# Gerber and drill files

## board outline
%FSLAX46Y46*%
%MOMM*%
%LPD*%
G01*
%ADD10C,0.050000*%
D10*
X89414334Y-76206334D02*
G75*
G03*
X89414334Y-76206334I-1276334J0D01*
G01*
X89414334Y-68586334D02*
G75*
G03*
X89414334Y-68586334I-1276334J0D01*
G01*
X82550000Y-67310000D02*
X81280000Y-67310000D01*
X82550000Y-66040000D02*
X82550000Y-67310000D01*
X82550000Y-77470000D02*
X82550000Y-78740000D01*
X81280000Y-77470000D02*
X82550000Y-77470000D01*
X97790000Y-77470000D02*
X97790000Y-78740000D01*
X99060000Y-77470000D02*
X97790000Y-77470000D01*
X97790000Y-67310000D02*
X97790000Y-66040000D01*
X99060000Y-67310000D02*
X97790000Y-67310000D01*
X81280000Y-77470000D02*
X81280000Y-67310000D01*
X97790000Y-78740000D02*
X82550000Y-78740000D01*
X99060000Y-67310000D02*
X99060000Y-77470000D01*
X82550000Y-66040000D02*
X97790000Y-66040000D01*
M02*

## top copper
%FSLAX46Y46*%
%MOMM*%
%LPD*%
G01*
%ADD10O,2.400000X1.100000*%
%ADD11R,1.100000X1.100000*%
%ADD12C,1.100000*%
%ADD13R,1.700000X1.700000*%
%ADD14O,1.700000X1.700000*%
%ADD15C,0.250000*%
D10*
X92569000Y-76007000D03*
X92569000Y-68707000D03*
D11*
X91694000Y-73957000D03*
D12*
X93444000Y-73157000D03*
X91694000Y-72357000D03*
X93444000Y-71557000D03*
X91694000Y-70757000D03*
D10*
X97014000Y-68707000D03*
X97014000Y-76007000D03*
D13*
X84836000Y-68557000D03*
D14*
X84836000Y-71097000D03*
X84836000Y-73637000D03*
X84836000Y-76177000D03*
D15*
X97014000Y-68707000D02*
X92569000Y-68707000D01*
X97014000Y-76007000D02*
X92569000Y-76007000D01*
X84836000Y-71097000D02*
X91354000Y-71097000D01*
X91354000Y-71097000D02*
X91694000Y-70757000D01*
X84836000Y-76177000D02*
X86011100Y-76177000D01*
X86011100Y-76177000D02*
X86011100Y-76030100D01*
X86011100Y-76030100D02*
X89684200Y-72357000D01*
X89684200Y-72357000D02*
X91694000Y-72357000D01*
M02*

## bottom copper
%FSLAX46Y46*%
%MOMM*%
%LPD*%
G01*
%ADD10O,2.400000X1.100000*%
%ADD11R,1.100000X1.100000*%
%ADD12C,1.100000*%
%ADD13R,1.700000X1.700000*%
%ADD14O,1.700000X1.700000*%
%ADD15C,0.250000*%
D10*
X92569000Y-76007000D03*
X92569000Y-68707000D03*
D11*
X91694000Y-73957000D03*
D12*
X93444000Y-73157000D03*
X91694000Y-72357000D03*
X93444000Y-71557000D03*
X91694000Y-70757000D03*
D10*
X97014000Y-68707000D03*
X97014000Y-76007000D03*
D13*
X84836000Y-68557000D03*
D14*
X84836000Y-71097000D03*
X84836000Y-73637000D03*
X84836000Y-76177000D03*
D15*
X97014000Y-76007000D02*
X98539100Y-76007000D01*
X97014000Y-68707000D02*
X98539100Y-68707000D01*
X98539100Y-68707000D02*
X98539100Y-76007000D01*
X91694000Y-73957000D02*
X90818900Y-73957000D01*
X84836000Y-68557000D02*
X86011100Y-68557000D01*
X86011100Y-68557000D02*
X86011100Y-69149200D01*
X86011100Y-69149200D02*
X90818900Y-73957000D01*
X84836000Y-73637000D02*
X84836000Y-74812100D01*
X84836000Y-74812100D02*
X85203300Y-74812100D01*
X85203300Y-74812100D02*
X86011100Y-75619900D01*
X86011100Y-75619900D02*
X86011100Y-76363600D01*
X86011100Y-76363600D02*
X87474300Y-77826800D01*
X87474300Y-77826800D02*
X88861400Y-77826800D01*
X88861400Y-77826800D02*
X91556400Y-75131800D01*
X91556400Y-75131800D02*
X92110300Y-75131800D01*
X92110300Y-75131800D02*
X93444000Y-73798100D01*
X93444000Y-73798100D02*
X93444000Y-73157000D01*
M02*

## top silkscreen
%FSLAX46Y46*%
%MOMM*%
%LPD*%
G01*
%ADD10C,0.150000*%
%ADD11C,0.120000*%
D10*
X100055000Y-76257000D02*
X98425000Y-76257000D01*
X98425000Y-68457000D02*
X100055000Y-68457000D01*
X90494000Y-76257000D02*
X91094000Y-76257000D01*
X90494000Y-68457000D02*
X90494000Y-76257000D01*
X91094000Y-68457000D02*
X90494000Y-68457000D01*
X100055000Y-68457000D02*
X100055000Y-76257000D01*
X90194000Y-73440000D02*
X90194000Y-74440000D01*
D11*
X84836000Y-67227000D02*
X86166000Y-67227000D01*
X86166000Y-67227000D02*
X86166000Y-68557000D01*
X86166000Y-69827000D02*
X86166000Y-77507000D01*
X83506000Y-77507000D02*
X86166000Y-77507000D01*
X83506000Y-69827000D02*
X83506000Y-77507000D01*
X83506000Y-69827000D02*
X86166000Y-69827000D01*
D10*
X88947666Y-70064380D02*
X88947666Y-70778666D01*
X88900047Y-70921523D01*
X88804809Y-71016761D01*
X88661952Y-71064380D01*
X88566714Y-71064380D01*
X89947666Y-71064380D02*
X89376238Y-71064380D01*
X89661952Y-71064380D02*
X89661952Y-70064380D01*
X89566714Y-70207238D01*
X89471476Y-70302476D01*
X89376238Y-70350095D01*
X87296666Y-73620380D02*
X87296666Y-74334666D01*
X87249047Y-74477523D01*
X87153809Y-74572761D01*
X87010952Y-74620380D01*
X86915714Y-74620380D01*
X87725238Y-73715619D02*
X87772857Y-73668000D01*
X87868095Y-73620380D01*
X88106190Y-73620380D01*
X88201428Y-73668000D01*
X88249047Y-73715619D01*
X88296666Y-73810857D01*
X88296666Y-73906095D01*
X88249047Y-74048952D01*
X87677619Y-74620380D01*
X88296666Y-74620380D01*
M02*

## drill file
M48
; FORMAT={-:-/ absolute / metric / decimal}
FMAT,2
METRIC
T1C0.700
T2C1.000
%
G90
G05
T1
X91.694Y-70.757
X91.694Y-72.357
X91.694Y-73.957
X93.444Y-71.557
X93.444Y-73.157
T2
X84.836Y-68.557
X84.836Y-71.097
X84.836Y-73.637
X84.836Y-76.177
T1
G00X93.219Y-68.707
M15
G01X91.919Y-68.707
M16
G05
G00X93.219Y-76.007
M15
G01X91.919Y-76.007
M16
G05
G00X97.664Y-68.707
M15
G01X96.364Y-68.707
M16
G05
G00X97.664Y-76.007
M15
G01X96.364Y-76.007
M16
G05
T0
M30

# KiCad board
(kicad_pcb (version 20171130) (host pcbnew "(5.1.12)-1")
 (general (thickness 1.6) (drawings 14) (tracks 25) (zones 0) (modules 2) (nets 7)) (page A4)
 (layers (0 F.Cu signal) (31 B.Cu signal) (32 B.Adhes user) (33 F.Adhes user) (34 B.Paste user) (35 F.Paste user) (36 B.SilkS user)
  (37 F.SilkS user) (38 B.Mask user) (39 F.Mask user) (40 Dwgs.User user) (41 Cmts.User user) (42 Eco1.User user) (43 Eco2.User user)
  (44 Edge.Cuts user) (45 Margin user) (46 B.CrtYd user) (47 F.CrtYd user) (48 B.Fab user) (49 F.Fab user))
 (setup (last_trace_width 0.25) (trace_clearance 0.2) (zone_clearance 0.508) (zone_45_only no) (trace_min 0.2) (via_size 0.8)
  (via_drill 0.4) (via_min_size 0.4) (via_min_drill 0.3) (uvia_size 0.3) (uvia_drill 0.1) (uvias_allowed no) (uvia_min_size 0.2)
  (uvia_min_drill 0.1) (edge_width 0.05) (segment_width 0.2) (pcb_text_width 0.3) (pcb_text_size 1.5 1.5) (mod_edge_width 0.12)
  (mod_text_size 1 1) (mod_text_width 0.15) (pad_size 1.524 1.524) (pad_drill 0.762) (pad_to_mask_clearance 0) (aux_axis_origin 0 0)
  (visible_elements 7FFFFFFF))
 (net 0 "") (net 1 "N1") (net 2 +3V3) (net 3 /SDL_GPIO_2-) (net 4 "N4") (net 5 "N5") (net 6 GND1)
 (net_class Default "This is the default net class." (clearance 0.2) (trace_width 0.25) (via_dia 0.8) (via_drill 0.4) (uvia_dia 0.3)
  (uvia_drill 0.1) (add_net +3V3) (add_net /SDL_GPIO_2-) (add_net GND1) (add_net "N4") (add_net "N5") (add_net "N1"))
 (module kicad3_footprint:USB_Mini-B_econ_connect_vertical (layer F.Cu) (at 99.06 72.281 90)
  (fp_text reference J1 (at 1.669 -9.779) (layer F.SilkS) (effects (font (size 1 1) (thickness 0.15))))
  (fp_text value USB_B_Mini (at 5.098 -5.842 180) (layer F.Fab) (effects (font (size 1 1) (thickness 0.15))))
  (fp_line (start -1.159 -8.866) (end -2.159 -8.866) (layer F.SilkS) (width 0.15))
  (fp_line (start 3.824 0.995) (end -3.976 0.995) (layer F.SilkS) (width 0.15))
  (fp_line (start 3.824 -7.966) (end 3.824 -8.566) (layer F.SilkS) (width 0.15))
  (fp_line (start 3.824 -8.566) (end -3.976 -8.566) (layer F.SilkS) (width 0.15))
  (fp_line (start -3.976 -8.566) (end -3.976 -7.966) (layer F.SilkS) (width 0.15))
  (fp_line (start 3.824 -0.635) (end 3.824 0.995) (layer F.SilkS) (width 0.15))
  (fp_line (start -3.976 0.995) (end -3.976 -0.635) (layer F.SilkS) (width 0.15))
  (pad 6 thru_hole oval (at -3.726 -6.491 270) (size 1.1 2.4) (drill oval 0.7 2) (layers *.Cu *.Mask) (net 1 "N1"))
  (pad 6 thru_hole oval (at 3.574 -6.491 270) (size 1.1 2.4) (drill oval 0.7 2) (layers *.Cu *.Mask) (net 1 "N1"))
  (pad 1 thru_hole rect (at -1.676 -7.366 270) (size 1.1 1.1) (drill 0.7) (layers *.Cu *.Mask) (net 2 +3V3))
  (pad 2 thru_hole circle (at -0.876 -5.616 270) (size 1.1 1.1) (drill 0.7) (layers *.Cu *.Mask) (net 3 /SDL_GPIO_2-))
  (pad 3 thru_hole circle (at -0.076 -7.366 270) (size 1.1 1.1) (drill 0.7) (layers *.Cu *.Mask) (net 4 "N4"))
  (pad 4 thru_hole circle (at 0.724 -5.616 270) (size 1.1 1.1) (drill 0.7) (layers *.Cu *.Mask) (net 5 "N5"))
  (pad 5 thru_hole circle (at 1.524 -7.366 270) (size 1.1 1.1) (drill 0.7) (layers *.Cu *.Mask) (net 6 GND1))
  (pad 6 thru_hole oval (at 3.574 -2.046 270) (size 1.1 2.4) (drill oval 0.7 2) (layers *.Cu *.Mask) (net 1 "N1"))
  (pad 6 thru_hole oval (at -3.726 -2.046 270) (size 1.1 2.4) (drill oval 0.7 2) (layers *.Cu *.Mask) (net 1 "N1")))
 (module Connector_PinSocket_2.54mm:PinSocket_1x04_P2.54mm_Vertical (layer F.Cu) (at 84.836 68.557)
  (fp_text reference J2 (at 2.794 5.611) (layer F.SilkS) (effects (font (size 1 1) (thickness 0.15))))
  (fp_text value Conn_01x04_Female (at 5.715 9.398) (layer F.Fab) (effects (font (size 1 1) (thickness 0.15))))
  (fp_line (start -1.33 1.27) (end 1.33 1.27) (layer F.SilkS) (width 0.12))
  (fp_line (start -1.33 1.27) (end -1.33 8.95) (layer F.SilkS) (width 0.12))
  (fp_line (start -1.33 8.95) (end 1.33 8.95) (layer F.SilkS) (width 0.12))
  (fp_line (start 1.33 1.27) (end 1.33 8.95) (layer F.SilkS) (width 0.12))
  (fp_line (start 1.33 -1.33) (end 1.33 0) (layer F.SilkS) (width 0.12))
  (fp_line (start 0 -1.33) (end 1.33 -1.33) (layer F.SilkS) (width 0.12))
  (pad 1 thru_hole rect (at 0 0) (size 1.7 1.7) (drill 1) (layers *.Cu *.Mask) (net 2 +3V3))
  (pad 2 thru_hole oval (at 0 2.54) (size 1.7 1.7) (drill 1) (layers *.Cu *.Mask) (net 6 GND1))
  (pad 3 thru_hole oval (at 0 5.08) (size 1.7 1.7) (drill 1) (layers *.Cu *.Mask) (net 3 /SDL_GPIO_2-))
  (pad 4 thru_hole oval (at 0 7.62) (size 1.7 1.7) (drill 1) (layers *.Cu *.Mask) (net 4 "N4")))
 (gr_circle (center 88.138 76.206334) (end 88.265 74.936334) (layer Edge.Cuts) (width 0.05))
 (gr_circle (center 88.138 68.586334) (end 88.265 67.316334) (layer Edge.Cuts) (width 0.05))
 (gr_line (start 82.55 67.31) (end 81.28 67.31) (layer Edge.Cuts) (width 0.05))
 (gr_line (start 82.55 66.04) (end 82.55 67.31) (layer Edge.Cuts) (width 0.05))
 (gr_line (start 82.55 77.47) (end 82.55 78.74) (layer Edge.Cuts) (width 0.05))
 (gr_line (start 81.28 77.47) (end 82.55 77.47) (layer Edge.Cuts) (width 0.05))
 (gr_line (start 97.79 77.47) (end 97.79 78.74) (layer Edge.Cuts) (width 0.05))
 (gr_line (start 99.06 77.47) (end 97.79 77.47) (layer Edge.Cuts) (width 0.05))
 (gr_line (start 97.79 67.31) (end 97.79 66.04) (layer Edge.Cuts) (width 0.05))
 (gr_line (start 99.06 67.31) (end 97.79 67.31) (layer Edge.Cuts) (width 0.05))
 (gr_line (start 81.28 77.47) (end 81.28 67.31) (layer Edge.Cuts) (width 0.05))
 (gr_line (start 97.79 78.74) (end 82.55 78.74) (layer Edge.Cuts) (width 0.05))
 (gr_line (start 99.06 67.31) (end 99.06 77.47) (layer Edge.Cuts) (width 0.05))
 (gr_line (start 82.55 66.04) (end 97.79 66.04) (layer Edge.Cuts) (width 0.05))
 (segment (start 97.014 76.007) (end 98.5391 76.007) (width 0.25) (layer B.Cu) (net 1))
 (segment (start 97.014 68.707) (end 98.5391 68.707) (width 0.25) (layer B.Cu) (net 1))
 (segment (start 98.5391 68.707) (end 98.5391 76.007) (width 0.25) (layer B.Cu) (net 1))
 (segment (start 97.014 68.707) (end 92.569 68.707) (width 0.25) (layer F.Cu) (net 1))
 (segment (start 97.014 76.007) (end 92.569 76.007) (width 0.25) (layer F.Cu) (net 1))
 (segment (start 91.694 73.957) (end 90.8189 73.957) (width 0.25) (layer B.Cu) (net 2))
 (segment (start 84.836 68.557) (end 86.0111 68.557) (width 0.25) (layer B.Cu) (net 2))
 (segment (start 86.0111 68.557) (end 86.0111 69.1492) (width 0.25) (layer B.Cu) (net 2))
 (segment (start 86.0111 69.1492) (end 90.8189 73.957) (width 0.25) (layer B.Cu) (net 2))
 (segment (start 84.836 71.097) (end 91.354 71.097) (width 0.25) (layer F.Cu) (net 6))
 (segment (start 91.354 71.097) (end 91.694 70.757) (width 0.25) (layer F.Cu) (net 6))
 (segment (start 84.836 76.177) (end 86.0111 76.177) (width 0.25) (layer F.Cu) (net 4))
 (segment (start 86.0111 76.177) (end 86.0111 76.0301) (width 0.25) (layer F.Cu) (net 4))
 (segment (start 86.0111 76.0301) (end 89.6842 72.357) (width 0.25) (layer F.Cu) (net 4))
 (segment (start 89.6842 72.357) (end 91.694 72.357) (width 0.25) (layer F.Cu) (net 4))
 (segment (start 84.836 73.637) (end 84.836 74.8121) (width 0.25) (layer B.Cu) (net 3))
 (segment (start 84.836 74.8121) (end 85.2033 74.8121) (width 0.25) (layer B.Cu) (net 3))
 (segment (start 85.2033 74.8121) (end 86.0111 75.6199) (width 0.25) (layer B.Cu) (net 3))
 (segment (start 86.0111 75.6199) (end 86.0111 76.3636) (width 0.25) (layer B.Cu) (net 3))
 (segment (start 86.0111 76.3636) (end 87.4743 77.8268) (width 0.25) (layer B.Cu) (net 3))
 (segment (start 87.4743 77.8268) (end 88.8614 77.8268) (width 0.25) (layer B.Cu) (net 3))
 (segment (start 88.8614 77.8268) (end 91.5564 75.1318) (width 0.25) (layer B.Cu) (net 3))
 (segment (start 91.5564 75.1318) (end 92.1103 75.1318) (width 0.25) (layer B.Cu) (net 3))
 (segment (start 92.1103 75.1318) (end 93.444 73.7981) (width 0.25) (layer B.Cu) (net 3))
 (segment (start 93.444 73.7981) (end 93.444 73.157) (width 0.25) (layer B.Cu) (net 3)))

